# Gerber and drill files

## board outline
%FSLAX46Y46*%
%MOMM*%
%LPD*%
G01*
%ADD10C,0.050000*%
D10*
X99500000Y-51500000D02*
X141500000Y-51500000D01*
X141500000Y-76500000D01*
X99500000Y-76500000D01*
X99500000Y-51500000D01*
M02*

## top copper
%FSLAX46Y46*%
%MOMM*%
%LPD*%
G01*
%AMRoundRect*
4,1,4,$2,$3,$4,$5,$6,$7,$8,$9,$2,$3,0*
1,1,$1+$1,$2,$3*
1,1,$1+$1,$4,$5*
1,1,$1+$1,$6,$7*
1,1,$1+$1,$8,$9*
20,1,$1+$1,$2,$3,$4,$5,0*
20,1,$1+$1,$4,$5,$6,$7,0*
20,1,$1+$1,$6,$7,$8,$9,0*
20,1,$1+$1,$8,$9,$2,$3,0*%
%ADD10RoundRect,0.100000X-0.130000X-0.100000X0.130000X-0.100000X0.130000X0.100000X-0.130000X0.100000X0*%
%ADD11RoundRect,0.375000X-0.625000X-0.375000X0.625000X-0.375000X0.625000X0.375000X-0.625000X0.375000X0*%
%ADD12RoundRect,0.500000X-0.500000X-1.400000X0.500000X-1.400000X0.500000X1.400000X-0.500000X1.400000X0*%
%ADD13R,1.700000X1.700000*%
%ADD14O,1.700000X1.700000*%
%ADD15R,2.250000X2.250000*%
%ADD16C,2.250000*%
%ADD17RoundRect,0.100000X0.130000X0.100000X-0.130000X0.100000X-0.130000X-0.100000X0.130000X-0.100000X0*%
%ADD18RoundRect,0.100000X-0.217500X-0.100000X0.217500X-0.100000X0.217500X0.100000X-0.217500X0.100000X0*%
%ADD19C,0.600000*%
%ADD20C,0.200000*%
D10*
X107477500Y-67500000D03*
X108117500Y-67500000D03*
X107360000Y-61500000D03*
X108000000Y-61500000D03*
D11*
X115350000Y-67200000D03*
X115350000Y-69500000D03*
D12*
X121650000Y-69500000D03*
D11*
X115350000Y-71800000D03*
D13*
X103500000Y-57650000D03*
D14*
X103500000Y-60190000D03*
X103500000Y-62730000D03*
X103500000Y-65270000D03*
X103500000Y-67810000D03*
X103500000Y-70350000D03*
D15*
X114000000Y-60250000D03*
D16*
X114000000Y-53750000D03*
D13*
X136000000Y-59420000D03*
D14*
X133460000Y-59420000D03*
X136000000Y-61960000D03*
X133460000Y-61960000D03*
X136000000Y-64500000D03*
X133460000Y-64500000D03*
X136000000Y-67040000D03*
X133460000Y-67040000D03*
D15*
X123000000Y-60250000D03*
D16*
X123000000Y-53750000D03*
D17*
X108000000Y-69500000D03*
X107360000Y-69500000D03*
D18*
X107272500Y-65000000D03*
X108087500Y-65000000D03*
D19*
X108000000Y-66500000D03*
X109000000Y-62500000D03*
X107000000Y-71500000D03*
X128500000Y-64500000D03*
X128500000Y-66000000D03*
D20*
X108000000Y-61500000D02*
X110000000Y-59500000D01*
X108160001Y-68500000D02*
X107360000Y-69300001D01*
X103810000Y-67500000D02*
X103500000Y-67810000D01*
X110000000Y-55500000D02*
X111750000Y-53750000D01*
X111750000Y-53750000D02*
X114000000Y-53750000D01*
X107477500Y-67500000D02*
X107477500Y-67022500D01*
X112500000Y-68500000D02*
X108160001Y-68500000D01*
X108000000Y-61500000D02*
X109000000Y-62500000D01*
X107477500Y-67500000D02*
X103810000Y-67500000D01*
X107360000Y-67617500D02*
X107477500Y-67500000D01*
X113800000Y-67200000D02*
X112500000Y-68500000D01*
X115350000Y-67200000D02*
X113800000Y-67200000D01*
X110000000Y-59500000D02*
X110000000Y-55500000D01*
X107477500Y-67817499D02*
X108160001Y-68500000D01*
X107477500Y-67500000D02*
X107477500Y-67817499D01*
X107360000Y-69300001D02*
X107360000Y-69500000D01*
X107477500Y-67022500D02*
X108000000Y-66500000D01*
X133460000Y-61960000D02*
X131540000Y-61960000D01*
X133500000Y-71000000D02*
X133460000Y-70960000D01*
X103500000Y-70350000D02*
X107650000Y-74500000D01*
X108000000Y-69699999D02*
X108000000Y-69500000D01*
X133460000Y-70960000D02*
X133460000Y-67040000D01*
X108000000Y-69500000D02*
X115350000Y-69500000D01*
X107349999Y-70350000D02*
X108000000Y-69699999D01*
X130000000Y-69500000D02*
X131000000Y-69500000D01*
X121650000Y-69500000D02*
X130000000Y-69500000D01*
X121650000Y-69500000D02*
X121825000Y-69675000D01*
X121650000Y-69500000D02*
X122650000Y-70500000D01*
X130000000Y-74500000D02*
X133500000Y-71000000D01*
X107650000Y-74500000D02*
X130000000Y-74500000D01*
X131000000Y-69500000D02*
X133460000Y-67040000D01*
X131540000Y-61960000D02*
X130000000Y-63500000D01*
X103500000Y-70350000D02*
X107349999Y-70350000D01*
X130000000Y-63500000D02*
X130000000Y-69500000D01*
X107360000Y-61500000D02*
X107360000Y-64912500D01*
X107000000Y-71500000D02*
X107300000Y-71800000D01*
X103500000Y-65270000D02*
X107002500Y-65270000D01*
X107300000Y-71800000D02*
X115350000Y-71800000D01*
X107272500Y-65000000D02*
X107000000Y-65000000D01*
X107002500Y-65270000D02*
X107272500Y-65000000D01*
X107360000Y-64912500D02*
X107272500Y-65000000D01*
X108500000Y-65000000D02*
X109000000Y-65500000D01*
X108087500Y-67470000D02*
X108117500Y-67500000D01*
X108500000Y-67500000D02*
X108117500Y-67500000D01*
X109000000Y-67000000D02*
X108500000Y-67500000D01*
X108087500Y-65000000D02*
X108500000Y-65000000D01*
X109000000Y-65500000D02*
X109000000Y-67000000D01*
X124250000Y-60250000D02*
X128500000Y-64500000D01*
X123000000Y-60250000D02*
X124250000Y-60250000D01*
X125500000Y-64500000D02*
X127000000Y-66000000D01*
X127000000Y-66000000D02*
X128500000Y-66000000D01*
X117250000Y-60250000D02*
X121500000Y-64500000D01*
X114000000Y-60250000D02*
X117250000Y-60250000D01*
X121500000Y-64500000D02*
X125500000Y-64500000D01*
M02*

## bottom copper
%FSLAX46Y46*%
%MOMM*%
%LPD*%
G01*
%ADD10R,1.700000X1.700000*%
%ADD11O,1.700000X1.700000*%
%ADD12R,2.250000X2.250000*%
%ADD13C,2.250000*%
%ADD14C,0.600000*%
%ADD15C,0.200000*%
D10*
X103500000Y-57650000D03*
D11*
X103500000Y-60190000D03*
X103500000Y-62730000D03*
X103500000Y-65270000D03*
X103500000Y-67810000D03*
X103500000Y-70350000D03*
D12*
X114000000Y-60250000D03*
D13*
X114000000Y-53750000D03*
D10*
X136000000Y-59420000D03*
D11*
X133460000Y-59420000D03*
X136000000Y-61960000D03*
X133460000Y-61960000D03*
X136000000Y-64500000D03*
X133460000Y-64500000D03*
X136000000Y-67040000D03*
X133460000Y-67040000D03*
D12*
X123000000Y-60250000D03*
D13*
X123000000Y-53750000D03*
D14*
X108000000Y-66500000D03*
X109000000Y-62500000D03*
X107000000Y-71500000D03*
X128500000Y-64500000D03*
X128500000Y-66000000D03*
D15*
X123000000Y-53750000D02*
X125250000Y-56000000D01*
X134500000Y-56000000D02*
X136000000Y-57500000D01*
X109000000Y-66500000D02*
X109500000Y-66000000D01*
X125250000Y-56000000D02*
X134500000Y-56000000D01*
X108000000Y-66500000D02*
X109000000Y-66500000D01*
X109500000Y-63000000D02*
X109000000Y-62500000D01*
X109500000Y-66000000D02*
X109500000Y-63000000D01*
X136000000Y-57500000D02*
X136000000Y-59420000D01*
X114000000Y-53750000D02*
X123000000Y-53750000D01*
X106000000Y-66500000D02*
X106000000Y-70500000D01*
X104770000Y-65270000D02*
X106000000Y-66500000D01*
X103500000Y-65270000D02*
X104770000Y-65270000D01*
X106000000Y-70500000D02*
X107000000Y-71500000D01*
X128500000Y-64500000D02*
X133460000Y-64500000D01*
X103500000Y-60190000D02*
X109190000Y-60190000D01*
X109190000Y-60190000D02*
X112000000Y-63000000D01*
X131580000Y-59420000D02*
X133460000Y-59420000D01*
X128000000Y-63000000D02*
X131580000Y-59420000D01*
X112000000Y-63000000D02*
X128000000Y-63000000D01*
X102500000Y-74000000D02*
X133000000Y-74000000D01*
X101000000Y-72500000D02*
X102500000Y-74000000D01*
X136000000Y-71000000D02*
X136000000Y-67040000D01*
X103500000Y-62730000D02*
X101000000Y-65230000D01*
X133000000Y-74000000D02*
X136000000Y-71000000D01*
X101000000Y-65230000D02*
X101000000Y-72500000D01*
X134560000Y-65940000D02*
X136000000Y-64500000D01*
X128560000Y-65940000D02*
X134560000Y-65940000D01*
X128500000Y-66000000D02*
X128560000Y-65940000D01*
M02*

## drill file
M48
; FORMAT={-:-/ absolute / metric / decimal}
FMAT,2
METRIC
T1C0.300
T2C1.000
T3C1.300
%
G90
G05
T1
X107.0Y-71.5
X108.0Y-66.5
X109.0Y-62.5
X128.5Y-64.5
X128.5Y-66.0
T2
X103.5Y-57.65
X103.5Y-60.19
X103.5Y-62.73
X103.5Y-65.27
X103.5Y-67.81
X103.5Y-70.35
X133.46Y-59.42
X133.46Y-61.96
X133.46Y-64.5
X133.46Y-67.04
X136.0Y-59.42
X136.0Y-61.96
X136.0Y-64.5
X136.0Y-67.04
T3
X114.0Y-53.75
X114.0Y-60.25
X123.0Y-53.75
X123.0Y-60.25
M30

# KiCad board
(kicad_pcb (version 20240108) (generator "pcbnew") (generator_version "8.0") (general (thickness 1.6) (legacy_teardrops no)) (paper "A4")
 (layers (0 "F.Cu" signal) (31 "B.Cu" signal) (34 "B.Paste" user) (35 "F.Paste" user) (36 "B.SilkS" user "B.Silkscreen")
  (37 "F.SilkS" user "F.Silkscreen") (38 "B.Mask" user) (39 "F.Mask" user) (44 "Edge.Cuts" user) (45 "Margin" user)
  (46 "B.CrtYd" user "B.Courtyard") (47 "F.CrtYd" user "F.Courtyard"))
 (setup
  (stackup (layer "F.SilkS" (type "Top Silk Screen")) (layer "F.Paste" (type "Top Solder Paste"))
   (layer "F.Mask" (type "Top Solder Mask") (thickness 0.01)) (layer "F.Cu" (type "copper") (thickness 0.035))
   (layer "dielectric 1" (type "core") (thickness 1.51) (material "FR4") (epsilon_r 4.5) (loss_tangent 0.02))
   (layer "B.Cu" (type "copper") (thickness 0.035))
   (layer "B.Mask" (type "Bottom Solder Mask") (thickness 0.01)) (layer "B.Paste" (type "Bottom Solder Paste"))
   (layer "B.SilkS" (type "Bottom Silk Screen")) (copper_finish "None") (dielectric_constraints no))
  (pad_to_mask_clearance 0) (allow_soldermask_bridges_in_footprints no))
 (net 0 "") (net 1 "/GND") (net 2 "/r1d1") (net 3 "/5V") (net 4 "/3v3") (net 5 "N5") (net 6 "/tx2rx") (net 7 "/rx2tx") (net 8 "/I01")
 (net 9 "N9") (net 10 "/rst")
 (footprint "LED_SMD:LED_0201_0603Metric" (layer "F.Cu") (at 107.7975 67.5)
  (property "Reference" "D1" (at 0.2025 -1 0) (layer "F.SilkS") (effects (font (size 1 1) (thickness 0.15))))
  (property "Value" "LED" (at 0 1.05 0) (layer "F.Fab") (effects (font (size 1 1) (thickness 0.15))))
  (pad "" smd roundrect (at -0.345 0) (size 0.318 0.36) (layers "F.Paste") (roundrect_rratio 0.25))
  (pad "" smd roundrect (at 0.345 0) (size 0.318 0.36) (layers "F.Paste") (roundrect_rratio 0.25))
  (pad "1" smd roundrect (at -0.32 0) (size 0.46 0.4) (layers "F.Cu" "F.Mask") (roundrect_rratio 0.25) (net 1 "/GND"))
  (pad "2" smd roundrect (at 0.32 0) (size 0.46 0.4) (layers "F.Cu" "F.Mask") (roundrect_rratio 0.25) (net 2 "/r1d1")))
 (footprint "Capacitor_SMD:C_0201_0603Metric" (layer "F.Cu") (at 107.68 61.5)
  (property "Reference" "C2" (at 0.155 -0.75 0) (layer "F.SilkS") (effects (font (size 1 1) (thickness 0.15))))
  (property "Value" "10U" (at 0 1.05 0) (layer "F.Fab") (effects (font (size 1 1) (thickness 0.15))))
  (pad "" smd roundrect (at -0.345 0) (size 0.318 0.36) (layers "F.Paste") (roundrect_rratio 0.25))
  (pad "" smd roundrect (at 0.345 0) (size 0.318 0.36) (layers "F.Paste") (roundrect_rratio 0.25))
  (pad "1" smd roundrect (at -0.32 0) (size 0.46 0.4) (layers "F.Cu" "F.Mask") (roundrect_rratio 0.25) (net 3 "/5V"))
  (pad "2" smd roundrect (at 0.32 0) (size 0.46 0.4) (layers "F.Cu" "F.Mask") (roundrect_rratio 0.25) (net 1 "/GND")))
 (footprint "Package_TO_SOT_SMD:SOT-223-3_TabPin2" (layer "F.Cu") (at 118.5 69.5)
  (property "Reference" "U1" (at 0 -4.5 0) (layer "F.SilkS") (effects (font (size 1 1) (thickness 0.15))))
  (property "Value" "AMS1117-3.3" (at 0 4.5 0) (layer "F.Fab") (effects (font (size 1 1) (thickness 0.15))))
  (pad "1" smd roundrect (at -3.15 -2.3) (size 2 1.5) (layers "F.Cu" "F.Paste" "F.Mask") (roundrect_rratio 0.25) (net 1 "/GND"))
  (pad "2" smd roundrect (at -3.15 0) (size 2 1.5) (layers "F.Cu" "F.Paste" "F.Mask") (roundrect_rratio 0.25) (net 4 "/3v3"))
  (pad "2" smd roundrect (at 3.15 0) (size 2 3.8) (layers "F.Cu" "F.Paste" "F.Mask") (roundrect_rratio 0.25) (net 4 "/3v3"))
  (pad "3" smd roundrect (at -3.15 2.3) (size 2 1.5) (layers "F.Cu" "F.Paste" "F.Mask") (roundrect_rratio 0.25) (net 3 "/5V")))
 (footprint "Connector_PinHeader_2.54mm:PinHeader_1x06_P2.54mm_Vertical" (layer "F.Cu") (at 103.5 57.65)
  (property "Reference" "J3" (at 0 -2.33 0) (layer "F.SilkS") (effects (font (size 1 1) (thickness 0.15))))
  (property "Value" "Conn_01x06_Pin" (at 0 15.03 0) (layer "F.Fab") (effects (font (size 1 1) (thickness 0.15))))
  (pad "1" thru_hole rect (at 0 0) (size 1.7 1.7) (drill 1) (layers "*.Cu" "*.Mask") (remove_unused_layers no) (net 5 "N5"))
  (pad "2" thru_hole oval (at 0 2.54) (size 1.7 1.7) (drill 1) (layers "*.Cu" "*.Mask") (remove_unused_layers no) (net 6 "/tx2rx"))
  (pad "3" thru_hole oval (at 0 5.08) (size 1.7 1.7) (drill 1) (layers "*.Cu" "*.Mask") (remove_unused_layers no) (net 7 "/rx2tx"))
  (pad "4" thru_hole oval (at 0 7.62) (size 1.7 1.7) (drill 1) (layers "*.Cu" "*.Mask") (remove_unused_layers no) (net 3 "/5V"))
  (pad "5" thru_hole oval (at 0 10.16) (size 1.7 1.7) (drill 1) (layers "*.Cu" "*.Mask") (remove_unused_layers no) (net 1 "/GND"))
  (pad "6" thru_hole oval (at 0 12.7) (size 1.7 1.7) (drill 1) (layers "*.Cu" "*.Mask") (remove_unused_layers no) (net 4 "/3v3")))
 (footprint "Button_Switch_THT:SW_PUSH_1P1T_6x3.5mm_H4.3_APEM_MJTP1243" (layer "F.Cu") (at 114 60.25 90)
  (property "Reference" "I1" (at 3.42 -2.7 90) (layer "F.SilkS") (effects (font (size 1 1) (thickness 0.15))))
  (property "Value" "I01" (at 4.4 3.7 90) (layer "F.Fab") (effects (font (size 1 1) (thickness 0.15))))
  (pad "1" thru_hole rect (at 0 0 180) (size 2.25 2.25) (drill 1.3) (layers "*.Cu" "*.Mask") (remove_unused_layers no) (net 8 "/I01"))
  (pad "2" thru_hole circle (at 6.5 0 180) (size 2.25 2.25) (drill 1.3) (layers "*.Cu" "*.Mask") (remove_unused_layers no) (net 1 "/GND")))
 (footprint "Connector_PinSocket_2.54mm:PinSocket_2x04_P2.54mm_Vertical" (layer "F.Cu") (at 136 59.42)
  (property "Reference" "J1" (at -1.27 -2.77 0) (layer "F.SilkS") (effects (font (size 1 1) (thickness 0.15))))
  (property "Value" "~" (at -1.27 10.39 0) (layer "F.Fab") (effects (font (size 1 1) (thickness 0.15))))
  (pad "1" thru_hole rect (at 0 0) (size 1.7 1.7) (drill 1) (layers "*.Cu" "*.Mask") (remove_unused_layers no) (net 1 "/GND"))
  (pad "2" thru_hole oval (at -2.54 0) (size 1.7 1.7) (drill 1) (layers "*.Cu" "*.Mask") (remove_unused_layers no) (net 6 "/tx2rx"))
  (pad "3" thru_hole oval (at 0 2.54) (size 1.7 1.7) (drill 1) (layers "*.Cu" "*.Mask") (remove_unused_layers no) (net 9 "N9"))
  (pad "4" thru_hole oval (at -2.54 2.54) (size 1.7 1.7) (drill 1) (layers "*.Cu" "*.Mask") (remove_unused_layers no) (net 4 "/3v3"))
  (pad "5" thru_hole oval (at 0 5.08) (size 1.7 1.7) (drill 1) (layers "*.Cu" "*.Mask") (remove_unused_layers no) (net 8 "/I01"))
  (pad "6" thru_hole oval (at -2.54 5.08) (size 1.7 1.7) (drill 1) (layers "*.Cu" "*.Mask") (remove_unused_layers no) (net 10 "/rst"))
  (pad "7" thru_hole oval (at 0 7.62) (size 1.7 1.7) (drill 1) (layers "*.Cu" "*.Mask") (remove_unused_layers no) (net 7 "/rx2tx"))
  (pad "8" thru_hole oval (at -2.54 7.62) (size 1.7 1.7) (drill 1) (layers "*.Cu" "*.Mask") (remove_unused_layers no) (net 4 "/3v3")))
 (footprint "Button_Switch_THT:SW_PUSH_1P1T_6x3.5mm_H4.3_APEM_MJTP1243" (layer "F.Cu") (at 123 60.25 90)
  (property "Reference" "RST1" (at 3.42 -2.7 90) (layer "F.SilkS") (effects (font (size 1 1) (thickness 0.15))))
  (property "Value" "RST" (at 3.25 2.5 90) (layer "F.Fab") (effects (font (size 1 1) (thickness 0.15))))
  (pad "1" thru_hole rect (at 0 0 180) (size 2.25 2.25) (drill 1.3) (layers "*.Cu" "*.Mask") (remove_unused_layers no) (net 10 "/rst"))
  (pad "2" thru_hole circle (at 6.5 0 180) (size 2.25 2.25) (drill 1.3) (layers "*.Cu" "*.Mask") (remove_unused_layers no) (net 1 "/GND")))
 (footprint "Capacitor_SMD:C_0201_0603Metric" (layer "F.Cu") (at 107.68 69.5 180)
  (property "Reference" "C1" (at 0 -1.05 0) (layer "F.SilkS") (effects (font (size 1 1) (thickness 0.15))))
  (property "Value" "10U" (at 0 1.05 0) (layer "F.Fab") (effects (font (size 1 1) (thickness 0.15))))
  (pad "" smd roundrect (at -0.345 0 180) (size 0.318 0.36) (layers "F.Paste") (roundrect_rratio 0.25))
  (pad "" smd roundrect (at 0.345 0 180) (size 0.318 0.36) (layers "F.Paste") (roundrect_rratio 0.25))
  (pad "1" smd roundrect (at -0.32 0 180) (size 0.46 0.4) (layers "F.Cu" "F.Mask") (roundrect_rratio 0.25) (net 4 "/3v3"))
  (pad "2" smd roundrect (at 0.32 0 180) (size 0.46 0.4) (layers "F.Cu" "F.Mask") (roundrect_rratio 0.25) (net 1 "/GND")))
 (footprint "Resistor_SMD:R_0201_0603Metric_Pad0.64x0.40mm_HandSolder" (layer "F.Cu") (at 107.68 65)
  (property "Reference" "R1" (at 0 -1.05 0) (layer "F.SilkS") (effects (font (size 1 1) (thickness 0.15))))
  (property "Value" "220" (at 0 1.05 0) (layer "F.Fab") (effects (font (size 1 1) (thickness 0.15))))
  (pad "" smd roundrect (at -0.4325 0) (size 0.458 0.36) (layers "F.Paste") (roundrect_rratio 0.25))
  (pad "" smd roundrect (at 0.4325 0) (size 0.458 0.36) (layers "F.Paste") (roundrect_rratio 0.25))
  (pad "1" smd roundrect (at -0.4075 0) (size 0.635 0.4) (layers "F.Cu" "F.Mask") (roundrect_rratio 0.25) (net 3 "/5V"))
  (pad "2" smd roundrect (at 0.4075 0) (size 0.635 0.4) (layers "F.Cu" "F.Mask") (roundrect_rratio 0.25) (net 2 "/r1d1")))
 (gr_rect (start 99.5 51.5) (end 141.5 76.5) (stroke (width 0.05) (type default)) (fill none) (layer "Edge.Cuts"))
 (segment (start 108 61.5) (end 110 59.5) (width 0.2) (layer "F.Cu") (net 1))
 (segment (start 108.160001 68.5) (end 107.36 69.300001) (width 0.2) (layer "F.Cu") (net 1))
 (segment (start 103.81 67.5) (end 103.5 67.81) (width 0.2) (layer "F.Cu") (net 1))
 (segment (start 110 55.5) (end 111.75 53.75) (width 0.2) (layer "F.Cu") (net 1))
 (segment (start 111.75 53.75) (end 114 53.75) (width 0.2) (layer "F.Cu") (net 1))
 (segment (start 107.4775 67.5) (end 107.4775 67.0225) (width 0.2) (layer "F.Cu") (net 1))
 (segment (start 112.5 68.5) (end 108.160001 68.5) (width 0.2) (layer "F.Cu") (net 1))
 (segment (start 108 61.5) (end 109 62.5) (width 0.2) (layer "F.Cu") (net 1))
 (segment (start 107.4775 67.5) (end 103.81 67.5) (width 0.2) (layer "F.Cu") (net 1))
 (segment (start 107.36 67.6175) (end 107.4775 67.5) (width 0.2) (layer "F.Cu") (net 1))
 (segment (start 113.8 67.2) (end 112.5 68.5) (width 0.2) (layer "F.Cu") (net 1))
 (segment (start 115.35 67.2) (end 113.8 67.2) (width 0.2) (layer "F.Cu") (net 1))
 (segment (start 110 59.5) (end 110 55.5) (width 0.2) (layer "F.Cu") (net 1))
 (segment (start 107.4775 67.817499) (end 108.160001 68.5) (width 0.2) (layer "F.Cu") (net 1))
 (segment (start 107.4775 67.5) (end 107.4775 67.817499) (width 0.2) (layer "F.Cu") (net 1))
 (segment (start 107.36 69.300001) (end 107.36 69.5) (width 0.2) (layer "F.Cu") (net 1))
 (segment (start 107.4775 67.0225) (end 108 66.5) (width 0.2) (layer "F.Cu") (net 1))
 (via (at 108 66.5) (size 0.6) (drill 0.3) (layers "F.Cu" "B.Cu") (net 1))
 (via (at 109 62.5) (size 0.6) (drill 0.3) (layers "F.Cu" "B.Cu") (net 1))
 (segment (start 123 53.75) (end 125.25 56) (width 0.2) (layer "B.Cu") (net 1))
 (segment (start 134.5 56) (end 136 57.5) (width 0.2) (layer "B.Cu") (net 1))
 (segment (start 109 66.5) (end 109.5 66) (width 0.2) (layer "B.Cu") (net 1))
 (segment (start 125.25 56) (end 134.5 56) (width 0.2) (layer "B.Cu") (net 1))
 (segment (start 108 66.5) (end 109 66.5) (width 0.2) (layer "B.Cu") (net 1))
 (segment (start 109.5 63) (end 109 62.5) (width 0.2) (layer "B.Cu") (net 1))
 (segment (start 109.5 66) (end 109.5 63) (width 0.2) (layer "B.Cu") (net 1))
 (segment (start 136 57.5) (end 136 59.42) (width 0.2) (layer "B.Cu") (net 1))
 (segment (start 114 53.75) (end 123 53.75) (width 0.2) (layer "B.Cu") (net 1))
 (segment (start 133.46 61.96) (end 131.54 61.96) (width 0.2) (layer "F.Cu") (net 4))
 (segment (start 133.5 71) (end 133.46 70.96) (width 0.2) (layer "F.Cu") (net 4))
 (segment (start 103.5 70.35) (end 107.65 74.5) (width 0.2) (layer "F.Cu") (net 4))
 (segment (start 108 69.699999) (end 108 69.5) (width 0.2) (layer "F.Cu") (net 4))
 (segment (start 133.46 70.96) (end 133.46 67.04) (width 0.2) (layer "F.Cu") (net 4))
 (segment (start 108 69.5) (end 115.35 69.5) (width 0.2) (layer "F.Cu") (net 4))
 (segment (start 107.349999 70.35) (end 108 69.699999) (width 0.2) (layer "F.Cu") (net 4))
 (segment (start 130 69.5) (end 131 69.5) (width 0.2) (layer "F.Cu") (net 4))
 (segment (start 121.65 69.5) (end 130 69.5) (width 0.2) (layer "F.Cu") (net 4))
 (segment (start 121.65 69.5) (end 121.825 69.675) (width 0.2) (layer "F.Cu") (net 4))
 (segment (start 121.65 69.5) (end 122.65 70.5) (width 0.2) (layer "F.Cu") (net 4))
 (segment (start 130 74.5) (end 133.5 71) (width 0.2) (layer "F.Cu") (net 4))
 (segment (start 107.65 74.5) (end 130 74.5) (width 0.2) (layer "F.Cu") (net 4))
 (segment (start 131 69.5) (end 133.46 67.04) (width 0.2) (layer "F.Cu") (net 4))
 (segment (start 131.54 61.96) (end 130 63.5) (width 0.2) (layer "F.Cu") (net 4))
 (segment (start 103.5 70.35) (end 107.349999 70.35) (width 0.2) (layer "F.Cu") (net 4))
 (segment (start 130 63.5) (end 130 69.5) (width 0.2) (layer "F.Cu") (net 4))
 (segment (start 107.36 61.5) (end 107.36 64.9125) (width 0.2) (layer "F.Cu") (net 3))
 (segment (start 107 71.5) (end 107.3 71.8) (width 0.2) (layer "F.Cu") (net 3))
 (segment (start 103.5 65.27) (end 107.0025 65.27) (width 0.2) (layer "F.Cu") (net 3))
 (segment (start 107.3 71.8) (end 115.35 71.8) (width 0.2) (layer "F.Cu") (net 3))
 (segment (start 107.2725 65) (end 107 65) (width 0.2) (layer "F.Cu") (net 3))
 (segment (start 107.0025 65.27) (end 107.2725 65) (width 0.2) (layer "F.Cu") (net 3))
 (segment (start 107.36 64.9125) (end 107.2725 65) (width 0.2) (layer "F.Cu") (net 3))
 (via (at 107 71.5) (size 0.6) (drill 0.3) (layers "F.Cu" "B.Cu") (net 3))
 (segment (start 106 66.5) (end 106 70.5) (width 0.2) (layer "B.Cu") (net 3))
 (segment (start 104.77 65.27) (end 106 66.5) (width 0.2) (layer "B.Cu") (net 3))
 (segment (start 103.5 65.27) (end 104.77 65.27) (width 0.2) (layer "B.Cu") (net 3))
 (segment (start 106 70.5) (end 107 71.5) (width 0.2) (layer "B.Cu") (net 3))
 (segment (start 108.5 65) (end 109 65.5) (width 0.2) (layer "F.Cu") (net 2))
 (segment (start 108.0875 67.47) (end 108.1175 67.5) (width 0.2) (layer "F.Cu") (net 2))
 (segment (start 108.5 67.5) (end 108.1175 67.5) (width 0.2) (layer "F.Cu") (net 2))
 (segment (start 109 67) (end 108.5 67.5) (width 0.2) (layer "F.Cu") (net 2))
 (segment (start 108.0875 65) (end 108.5 65) (width 0.2) (layer "F.Cu") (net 2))
 (segment (start 109 65.5) (end 109 67) (width 0.2) (layer "F.Cu") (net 2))
 (segment (start 124.25 60.25) (end 128.5 64.5) (width 0.2) (layer "F.Cu") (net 10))
 (segment (start 123 60.25) (end 124.25 60.25) (width 0.2) (layer "F.Cu") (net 10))
 (via (at 128.5 64.5) (size 0.6) (drill 0.3) (layers "F.Cu" "B.Cu") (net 10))
 (segment (start 128.5 64.5) (end 133.46 64.5) (width 0.2) (layer "B.Cu") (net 10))
 (segment (start 103.5 60.19) (end 109.19 60.19) (width 0.2) (layer "B.Cu") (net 6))
 (segment (start 109.19 60.19) (end 112 63) (width 0.2) (layer "B.Cu") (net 6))
 (segment (start 131.58 59.42) (end 133.46 59.42) (width 0.2) (layer "B.Cu") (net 6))
 (segment (start 128 63) (end 131.58 59.42) (width 0.2) (layer "B.Cu") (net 6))
 (segment (start 112 63) (end 128 63) (width 0.2) (layer "B.Cu") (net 6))
 (segment (start 102.5 74) (end 133 74) (width 0.2) (layer "B.Cu") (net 7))
 (segment (start 101 72.5) (end 102.5 74) (width 0.2) (layer "B.Cu") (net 7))
 (segment (start 136 71) (end 136 67.04) (width 0.2) (layer "B.Cu") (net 7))
 (segment (start 103.5 62.73) (end 101 65.23) (width 0.2) (layer "B.Cu") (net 7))
 (segment (start 133 74) (end 136 71) (width 0.2) (layer "B.Cu") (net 7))
 (segment (start 101 65.23) (end 101 72.5) (width 0.2) (layer "B.Cu") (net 7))
 (segment (start 125.5 64.5) (end 127 66) (width 0.2) (layer "F.Cu") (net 8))
 (segment (start 127 66) (end 128.5 66) (width 0.2) (layer "F.Cu") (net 8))
 (segment (start 117.25 60.25) (end 121.5 64.5) (width 0.2) (layer "F.Cu") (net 8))
 (segment (start 114 60.25) (end 117.25 60.25) (width 0.2) (layer "F.Cu") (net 8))
 (segment (start 121.5 64.5) (end 125.5 64.5) (width 0.2) (layer "F.Cu") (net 8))
 (via (at 128.5 66) (size 0.6) (drill 0.3) (layers "F.Cu" "B.Cu") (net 8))
 (segment (start 134.56 65.94) (end 136 64.5) (width 0.2) (layer "B.Cu") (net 8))
 (segment (start 128.56 65.94) (end 134.56 65.94) (width 0.2) (layer "B.Cu") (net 8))
 (segment (start 128.5 66) (end 128.56 65.94) (width 0.2) (layer "B.Cu") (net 8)))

